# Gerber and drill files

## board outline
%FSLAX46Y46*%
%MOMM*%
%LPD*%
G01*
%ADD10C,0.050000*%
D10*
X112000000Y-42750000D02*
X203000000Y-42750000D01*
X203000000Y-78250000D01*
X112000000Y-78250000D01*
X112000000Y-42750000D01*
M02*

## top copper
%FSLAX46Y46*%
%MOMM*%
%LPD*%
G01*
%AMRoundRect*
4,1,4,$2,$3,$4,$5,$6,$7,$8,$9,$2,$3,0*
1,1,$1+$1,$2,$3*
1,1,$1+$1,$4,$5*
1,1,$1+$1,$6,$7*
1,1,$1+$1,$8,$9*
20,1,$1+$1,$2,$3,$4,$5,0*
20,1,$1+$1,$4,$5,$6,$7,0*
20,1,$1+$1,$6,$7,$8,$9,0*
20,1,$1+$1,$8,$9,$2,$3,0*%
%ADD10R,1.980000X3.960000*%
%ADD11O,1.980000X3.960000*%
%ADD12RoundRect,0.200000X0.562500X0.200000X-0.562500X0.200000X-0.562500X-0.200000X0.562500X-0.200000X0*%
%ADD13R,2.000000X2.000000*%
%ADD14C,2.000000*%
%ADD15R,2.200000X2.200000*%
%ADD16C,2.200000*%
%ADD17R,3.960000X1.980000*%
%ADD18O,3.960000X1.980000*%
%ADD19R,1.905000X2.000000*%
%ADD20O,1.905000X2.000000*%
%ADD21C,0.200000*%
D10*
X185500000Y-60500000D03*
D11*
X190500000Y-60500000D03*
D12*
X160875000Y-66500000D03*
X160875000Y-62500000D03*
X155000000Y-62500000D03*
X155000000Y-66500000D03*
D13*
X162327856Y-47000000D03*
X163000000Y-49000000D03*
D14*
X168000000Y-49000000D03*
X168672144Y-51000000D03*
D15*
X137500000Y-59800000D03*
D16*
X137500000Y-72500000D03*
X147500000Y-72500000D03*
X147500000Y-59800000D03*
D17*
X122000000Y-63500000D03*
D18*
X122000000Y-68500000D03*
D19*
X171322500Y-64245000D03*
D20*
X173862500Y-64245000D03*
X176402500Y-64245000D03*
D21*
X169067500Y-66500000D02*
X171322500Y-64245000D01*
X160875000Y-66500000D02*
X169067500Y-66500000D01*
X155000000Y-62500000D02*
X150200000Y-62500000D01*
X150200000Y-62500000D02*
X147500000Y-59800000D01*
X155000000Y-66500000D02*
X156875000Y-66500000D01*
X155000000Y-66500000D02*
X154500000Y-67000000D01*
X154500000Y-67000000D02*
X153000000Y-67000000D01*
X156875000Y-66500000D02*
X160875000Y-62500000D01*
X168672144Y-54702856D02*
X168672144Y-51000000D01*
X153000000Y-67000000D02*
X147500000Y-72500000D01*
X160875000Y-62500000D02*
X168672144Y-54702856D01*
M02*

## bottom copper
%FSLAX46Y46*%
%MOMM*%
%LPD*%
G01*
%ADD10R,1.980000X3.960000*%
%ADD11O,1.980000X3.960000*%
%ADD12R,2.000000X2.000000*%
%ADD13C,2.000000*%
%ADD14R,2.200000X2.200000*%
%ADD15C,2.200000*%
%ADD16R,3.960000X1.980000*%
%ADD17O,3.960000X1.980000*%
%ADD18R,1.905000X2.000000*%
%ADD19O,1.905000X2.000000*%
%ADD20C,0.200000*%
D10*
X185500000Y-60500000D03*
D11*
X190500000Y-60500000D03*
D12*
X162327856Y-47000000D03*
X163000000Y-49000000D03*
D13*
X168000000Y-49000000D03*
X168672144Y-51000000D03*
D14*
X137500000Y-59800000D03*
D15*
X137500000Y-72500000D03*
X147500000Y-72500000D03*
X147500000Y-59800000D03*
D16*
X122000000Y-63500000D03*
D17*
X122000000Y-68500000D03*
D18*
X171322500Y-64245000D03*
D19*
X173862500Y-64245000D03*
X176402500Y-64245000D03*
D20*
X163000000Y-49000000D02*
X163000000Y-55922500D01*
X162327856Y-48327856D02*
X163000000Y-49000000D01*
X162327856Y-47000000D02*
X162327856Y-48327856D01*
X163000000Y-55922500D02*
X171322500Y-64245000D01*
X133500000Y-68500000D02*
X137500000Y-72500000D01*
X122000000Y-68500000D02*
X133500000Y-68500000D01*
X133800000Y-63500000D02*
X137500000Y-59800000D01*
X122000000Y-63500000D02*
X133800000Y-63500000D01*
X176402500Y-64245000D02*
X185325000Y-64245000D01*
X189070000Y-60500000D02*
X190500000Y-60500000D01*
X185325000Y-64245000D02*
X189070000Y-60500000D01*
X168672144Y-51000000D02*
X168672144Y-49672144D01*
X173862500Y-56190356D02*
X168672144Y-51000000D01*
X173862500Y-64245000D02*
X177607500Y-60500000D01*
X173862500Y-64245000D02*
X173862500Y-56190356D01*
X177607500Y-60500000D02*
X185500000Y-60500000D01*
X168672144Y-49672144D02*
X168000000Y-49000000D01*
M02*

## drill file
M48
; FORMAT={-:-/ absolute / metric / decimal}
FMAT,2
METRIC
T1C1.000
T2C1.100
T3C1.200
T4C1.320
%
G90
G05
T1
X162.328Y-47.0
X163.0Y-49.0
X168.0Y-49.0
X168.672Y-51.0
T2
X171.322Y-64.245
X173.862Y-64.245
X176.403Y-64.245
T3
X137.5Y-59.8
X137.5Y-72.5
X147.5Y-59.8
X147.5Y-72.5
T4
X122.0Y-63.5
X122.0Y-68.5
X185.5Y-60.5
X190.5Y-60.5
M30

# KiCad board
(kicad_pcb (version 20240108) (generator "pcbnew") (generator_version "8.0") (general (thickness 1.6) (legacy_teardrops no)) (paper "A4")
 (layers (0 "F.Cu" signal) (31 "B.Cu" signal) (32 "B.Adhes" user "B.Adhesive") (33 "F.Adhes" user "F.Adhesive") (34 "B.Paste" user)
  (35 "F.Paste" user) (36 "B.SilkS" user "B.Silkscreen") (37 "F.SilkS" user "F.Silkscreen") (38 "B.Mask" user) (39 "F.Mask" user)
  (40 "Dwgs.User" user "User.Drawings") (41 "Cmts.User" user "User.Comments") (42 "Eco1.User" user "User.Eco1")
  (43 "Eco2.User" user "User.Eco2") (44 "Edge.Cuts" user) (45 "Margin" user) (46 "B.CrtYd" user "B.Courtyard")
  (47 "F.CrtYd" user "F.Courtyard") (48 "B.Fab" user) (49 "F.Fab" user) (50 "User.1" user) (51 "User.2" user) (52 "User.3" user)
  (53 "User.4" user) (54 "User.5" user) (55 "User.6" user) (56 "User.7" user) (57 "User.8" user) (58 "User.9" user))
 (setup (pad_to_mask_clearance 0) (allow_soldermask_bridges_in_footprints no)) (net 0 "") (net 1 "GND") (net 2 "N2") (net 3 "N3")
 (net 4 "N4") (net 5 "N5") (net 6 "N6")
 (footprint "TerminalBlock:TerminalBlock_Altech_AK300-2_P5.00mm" (layer "F.Cu") (at 185.5 60.5)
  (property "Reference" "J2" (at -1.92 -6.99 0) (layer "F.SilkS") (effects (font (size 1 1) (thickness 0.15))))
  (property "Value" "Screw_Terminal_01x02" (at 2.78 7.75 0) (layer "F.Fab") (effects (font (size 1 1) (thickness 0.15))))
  (pad "1" thru_hole rect (at 0 0) (size 1.98 3.96) (drill 1.32) (layers "*.Cu" "*.Mask") (remove_unused_layers no) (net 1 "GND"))
  (pad "2" thru_hole oval (at 5 0) (size 1.98 3.96) (drill 1.32) (layers "*.Cu" "*.Mask") (remove_unused_layers no) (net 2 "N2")))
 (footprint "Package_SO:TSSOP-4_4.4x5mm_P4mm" (layer "F.Cu") (at 157.9375 64.5 180)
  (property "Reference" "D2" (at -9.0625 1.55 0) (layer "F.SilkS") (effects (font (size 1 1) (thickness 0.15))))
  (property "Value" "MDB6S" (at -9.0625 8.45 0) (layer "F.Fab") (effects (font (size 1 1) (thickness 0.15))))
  (pad "1" smd roundrect (at -2.9375 -2 180) (size 1.525 0.8) (layers "F.Cu" "F.Paste" "F.Mask") (roundrect_rratio 0.25) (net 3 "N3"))
  (pad "2" smd roundrect (at -2.9375 2 180) (size 1.525 0.8) (layers "F.Cu" "F.Paste" "F.Mask") (roundrect_rratio 0.25) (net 1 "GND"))
  (pad "3" smd roundrect (at 2.9375 2 180) (size 1.525 0.8) (layers "F.Cu" "F.Paste" "F.Mask") (roundrect_rratio 0.25) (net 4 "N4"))
  (pad "4" smd roundrect (at 2.9375 -2 180) (size 1.525 0.8) (layers "F.Cu" "F.Paste" "F.Mask") (roundrect_rratio 0.25) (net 1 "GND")))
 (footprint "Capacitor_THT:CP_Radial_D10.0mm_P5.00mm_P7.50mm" (layer "F.Cu") (at 163 49)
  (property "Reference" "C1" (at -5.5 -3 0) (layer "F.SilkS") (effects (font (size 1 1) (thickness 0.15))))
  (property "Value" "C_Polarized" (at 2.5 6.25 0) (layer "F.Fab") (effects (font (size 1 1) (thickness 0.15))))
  (pad "1" thru_hole rect (at -0.672144 -2) (size 2 2) (drill 1) (layers "*.Cu" "*.Mask") (remove_unused_layers no) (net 3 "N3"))
  (pad "1" thru_hole rect (at 0 0) (size 2 2) (drill 1) (layers "*.Cu" "*.Mask") (remove_unused_layers no) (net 3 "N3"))
  (pad "2" thru_hole circle (at 5 0) (size 2 2) (drill 1) (layers "*.Cu" "*.Mask") (remove_unused_layers no) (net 1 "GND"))
  (pad "2" thru_hole circle (at 5.672144 2) (size 2 2) (drill 1) (layers "*.Cu" "*.Mask") (remove_unused_layers no) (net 1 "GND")))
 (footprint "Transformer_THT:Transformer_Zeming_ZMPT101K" (layer "F.Cu") (at 137.5 59.8)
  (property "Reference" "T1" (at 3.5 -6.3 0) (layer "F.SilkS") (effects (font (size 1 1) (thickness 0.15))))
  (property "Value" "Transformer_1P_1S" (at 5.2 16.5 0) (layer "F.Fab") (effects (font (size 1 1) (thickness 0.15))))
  (pad "1" thru_hole rect (at 0 0) (size 2.2 2.2) (drill 1.2) (layers "*.Cu" "*.Mask") (remove_unused_layers no) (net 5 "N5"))
  (pad "2" thru_hole circle (at 0 12.7) (size 2.2 2.2) (drill 1.2) (layers "*.Cu" "*.Mask") (remove_unused_layers no) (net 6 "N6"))
  (pad "3" thru_hole circle (at 10 12.7) (size 2.2 2.2) (drill 1.2) (layers "*.Cu" "*.Mask") (remove_unused_layers no) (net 1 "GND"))
  (pad "4" thru_hole circle (at 10 0) (size 2.2 2.2) (drill 1.2) (layers "*.Cu" "*.Mask") (remove_unused_layers no) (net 4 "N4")))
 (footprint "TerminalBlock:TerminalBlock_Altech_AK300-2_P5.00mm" (layer "F.Cu") (at 122 63.5 -90)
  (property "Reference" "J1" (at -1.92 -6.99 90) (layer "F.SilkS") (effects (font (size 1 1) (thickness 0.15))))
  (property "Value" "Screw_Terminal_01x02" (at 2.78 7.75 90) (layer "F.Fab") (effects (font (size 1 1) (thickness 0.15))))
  (pad "1" thru_hole rect (at 0 0 270) (size 1.98 3.96) (drill 1.32) (layers "*.Cu" "*.Mask") (remove_unused_layers no) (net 5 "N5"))
  (pad "2" thru_hole oval (at 5 0 270) (size 1.98 3.96) (drill 1.32) (layers "*.Cu" "*.Mask") (remove_unused_layers no) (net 6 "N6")))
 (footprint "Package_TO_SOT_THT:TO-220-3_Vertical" (layer "F.Cu") (at 171.3225 64.245)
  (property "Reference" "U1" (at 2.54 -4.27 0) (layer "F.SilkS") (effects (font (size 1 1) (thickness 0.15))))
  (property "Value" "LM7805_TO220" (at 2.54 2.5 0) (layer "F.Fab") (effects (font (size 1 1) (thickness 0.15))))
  (pad "1" thru_hole rect (at 0 0) (size 1.905 2) (drill 1.1) (layers "*.Cu" "*.Mask") (remove_unused_layers no) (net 3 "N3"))
  (pad "2" thru_hole oval (at 2.54 0) (size 1.905 2) (drill 1.1) (layers "*.Cu" "*.Mask") (remove_unused_layers no) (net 1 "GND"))
  (pad "3" thru_hole oval (at 5.08 0) (size 1.905 2) (drill 1.1) (layers "*.Cu" "*.Mask") (remove_unused_layers no) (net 2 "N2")))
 (gr_rect (start 112 42.75) (end 203 78.25) (stroke (width 0.05) (type default)) (fill none) (layer "Edge.Cuts"))
 (segment (start 169.0675 66.5) (end 171.3225 64.245) (width 0.2) (layer "F.Cu") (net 3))
 (segment (start 160.875 66.5) (end 169.0675 66.5) (width 0.2) (layer "F.Cu") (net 3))
 (segment (start 163 49) (end 163 55.9225) (width 0.2) (layer "B.Cu") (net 3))
 (segment (start 162.327856 48.327856) (end 163 49) (width 0.2) (layer "B.Cu") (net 3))
 (segment (start 162.327856 47) (end 162.327856 48.327856) (width 0.2) (layer "B.Cu") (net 3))
 (segment (start 163 55.9225) (end 171.3225 64.245) (width 0.2) (layer "B.Cu") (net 3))
 (segment (start 155 62.5) (end 150.2 62.5) (width 0.2) (layer "F.Cu") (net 4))
 (segment (start 150.2 62.5) (end 147.5 59.8) (width 0.2) (layer "F.Cu") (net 4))
 (segment (start 133.5 68.5) (end 137.5 72.5) (width 0.2) (layer "B.Cu") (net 6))
 (segment (start 122 68.5) (end 133.5 68.5) (width 0.2) (layer "B.Cu") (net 6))
 (segment (start 133.8 63.5) (end 137.5 59.8) (width 0.2) (layer "B.Cu") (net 5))
 (segment (start 122 63.5) (end 133.8 63.5) (width 0.2) (layer "B.Cu") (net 5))
 (segment (start 176.4025 64.245) (end 185.325 64.245) (width 0.2) (layer "B.Cu") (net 2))
 (segment (start 189.07 60.5) (end 190.5 60.5) (width 0.2) (layer "B.Cu") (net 2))
 (segment (start 185.325 64.245) (end 189.07 60.5) (width 0.2) (layer "B.Cu") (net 2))
 (segment (start 155 66.5) (end 156.875 66.5) (width 0.2) (layer "F.Cu") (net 1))
 (segment (start 155 66.5) (end 154.5 67) (width 0.2) (layer "F.Cu") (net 1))
 (segment (start 154.5 67) (end 153 67) (width 0.2) (layer "F.Cu") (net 1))
 (segment (start 156.875 66.5) (end 160.875 62.5) (width 0.2) (layer "F.Cu") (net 1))
 (segment (start 168.672144 54.702856) (end 168.672144 51) (width 0.2) (layer "F.Cu") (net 1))
 (segment (start 153 67) (end 147.5 72.5) (width 0.2) (layer "F.Cu") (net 1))
 (segment (start 160.875 62.5) (end 168.672144 54.702856) (width 0.2) (layer "F.Cu") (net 1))
 (segment (start 168.672144 51) (end 168.672144 49.672144) (width 0.2) (layer "B.Cu") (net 1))
 (segment (start 173.8625 56.190356) (end 168.672144 51) (width 0.2) (layer "B.Cu") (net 1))
 (segment (start 173.8625 64.245) (end 177.6075 60.5) (width 0.2) (layer "B.Cu") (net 1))
 (segment (start 173.8625 64.245) (end 173.8625 56.190356) (width 0.2) (layer "B.Cu") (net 1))
 (segment (start 177.6075 60.5) (end 185.5 60.5) (width 0.2) (layer "B.Cu") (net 1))
 (segment (start 168.672144 49.672144) (end 168 49) (width 0.2) (layer "B.Cu") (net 1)))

